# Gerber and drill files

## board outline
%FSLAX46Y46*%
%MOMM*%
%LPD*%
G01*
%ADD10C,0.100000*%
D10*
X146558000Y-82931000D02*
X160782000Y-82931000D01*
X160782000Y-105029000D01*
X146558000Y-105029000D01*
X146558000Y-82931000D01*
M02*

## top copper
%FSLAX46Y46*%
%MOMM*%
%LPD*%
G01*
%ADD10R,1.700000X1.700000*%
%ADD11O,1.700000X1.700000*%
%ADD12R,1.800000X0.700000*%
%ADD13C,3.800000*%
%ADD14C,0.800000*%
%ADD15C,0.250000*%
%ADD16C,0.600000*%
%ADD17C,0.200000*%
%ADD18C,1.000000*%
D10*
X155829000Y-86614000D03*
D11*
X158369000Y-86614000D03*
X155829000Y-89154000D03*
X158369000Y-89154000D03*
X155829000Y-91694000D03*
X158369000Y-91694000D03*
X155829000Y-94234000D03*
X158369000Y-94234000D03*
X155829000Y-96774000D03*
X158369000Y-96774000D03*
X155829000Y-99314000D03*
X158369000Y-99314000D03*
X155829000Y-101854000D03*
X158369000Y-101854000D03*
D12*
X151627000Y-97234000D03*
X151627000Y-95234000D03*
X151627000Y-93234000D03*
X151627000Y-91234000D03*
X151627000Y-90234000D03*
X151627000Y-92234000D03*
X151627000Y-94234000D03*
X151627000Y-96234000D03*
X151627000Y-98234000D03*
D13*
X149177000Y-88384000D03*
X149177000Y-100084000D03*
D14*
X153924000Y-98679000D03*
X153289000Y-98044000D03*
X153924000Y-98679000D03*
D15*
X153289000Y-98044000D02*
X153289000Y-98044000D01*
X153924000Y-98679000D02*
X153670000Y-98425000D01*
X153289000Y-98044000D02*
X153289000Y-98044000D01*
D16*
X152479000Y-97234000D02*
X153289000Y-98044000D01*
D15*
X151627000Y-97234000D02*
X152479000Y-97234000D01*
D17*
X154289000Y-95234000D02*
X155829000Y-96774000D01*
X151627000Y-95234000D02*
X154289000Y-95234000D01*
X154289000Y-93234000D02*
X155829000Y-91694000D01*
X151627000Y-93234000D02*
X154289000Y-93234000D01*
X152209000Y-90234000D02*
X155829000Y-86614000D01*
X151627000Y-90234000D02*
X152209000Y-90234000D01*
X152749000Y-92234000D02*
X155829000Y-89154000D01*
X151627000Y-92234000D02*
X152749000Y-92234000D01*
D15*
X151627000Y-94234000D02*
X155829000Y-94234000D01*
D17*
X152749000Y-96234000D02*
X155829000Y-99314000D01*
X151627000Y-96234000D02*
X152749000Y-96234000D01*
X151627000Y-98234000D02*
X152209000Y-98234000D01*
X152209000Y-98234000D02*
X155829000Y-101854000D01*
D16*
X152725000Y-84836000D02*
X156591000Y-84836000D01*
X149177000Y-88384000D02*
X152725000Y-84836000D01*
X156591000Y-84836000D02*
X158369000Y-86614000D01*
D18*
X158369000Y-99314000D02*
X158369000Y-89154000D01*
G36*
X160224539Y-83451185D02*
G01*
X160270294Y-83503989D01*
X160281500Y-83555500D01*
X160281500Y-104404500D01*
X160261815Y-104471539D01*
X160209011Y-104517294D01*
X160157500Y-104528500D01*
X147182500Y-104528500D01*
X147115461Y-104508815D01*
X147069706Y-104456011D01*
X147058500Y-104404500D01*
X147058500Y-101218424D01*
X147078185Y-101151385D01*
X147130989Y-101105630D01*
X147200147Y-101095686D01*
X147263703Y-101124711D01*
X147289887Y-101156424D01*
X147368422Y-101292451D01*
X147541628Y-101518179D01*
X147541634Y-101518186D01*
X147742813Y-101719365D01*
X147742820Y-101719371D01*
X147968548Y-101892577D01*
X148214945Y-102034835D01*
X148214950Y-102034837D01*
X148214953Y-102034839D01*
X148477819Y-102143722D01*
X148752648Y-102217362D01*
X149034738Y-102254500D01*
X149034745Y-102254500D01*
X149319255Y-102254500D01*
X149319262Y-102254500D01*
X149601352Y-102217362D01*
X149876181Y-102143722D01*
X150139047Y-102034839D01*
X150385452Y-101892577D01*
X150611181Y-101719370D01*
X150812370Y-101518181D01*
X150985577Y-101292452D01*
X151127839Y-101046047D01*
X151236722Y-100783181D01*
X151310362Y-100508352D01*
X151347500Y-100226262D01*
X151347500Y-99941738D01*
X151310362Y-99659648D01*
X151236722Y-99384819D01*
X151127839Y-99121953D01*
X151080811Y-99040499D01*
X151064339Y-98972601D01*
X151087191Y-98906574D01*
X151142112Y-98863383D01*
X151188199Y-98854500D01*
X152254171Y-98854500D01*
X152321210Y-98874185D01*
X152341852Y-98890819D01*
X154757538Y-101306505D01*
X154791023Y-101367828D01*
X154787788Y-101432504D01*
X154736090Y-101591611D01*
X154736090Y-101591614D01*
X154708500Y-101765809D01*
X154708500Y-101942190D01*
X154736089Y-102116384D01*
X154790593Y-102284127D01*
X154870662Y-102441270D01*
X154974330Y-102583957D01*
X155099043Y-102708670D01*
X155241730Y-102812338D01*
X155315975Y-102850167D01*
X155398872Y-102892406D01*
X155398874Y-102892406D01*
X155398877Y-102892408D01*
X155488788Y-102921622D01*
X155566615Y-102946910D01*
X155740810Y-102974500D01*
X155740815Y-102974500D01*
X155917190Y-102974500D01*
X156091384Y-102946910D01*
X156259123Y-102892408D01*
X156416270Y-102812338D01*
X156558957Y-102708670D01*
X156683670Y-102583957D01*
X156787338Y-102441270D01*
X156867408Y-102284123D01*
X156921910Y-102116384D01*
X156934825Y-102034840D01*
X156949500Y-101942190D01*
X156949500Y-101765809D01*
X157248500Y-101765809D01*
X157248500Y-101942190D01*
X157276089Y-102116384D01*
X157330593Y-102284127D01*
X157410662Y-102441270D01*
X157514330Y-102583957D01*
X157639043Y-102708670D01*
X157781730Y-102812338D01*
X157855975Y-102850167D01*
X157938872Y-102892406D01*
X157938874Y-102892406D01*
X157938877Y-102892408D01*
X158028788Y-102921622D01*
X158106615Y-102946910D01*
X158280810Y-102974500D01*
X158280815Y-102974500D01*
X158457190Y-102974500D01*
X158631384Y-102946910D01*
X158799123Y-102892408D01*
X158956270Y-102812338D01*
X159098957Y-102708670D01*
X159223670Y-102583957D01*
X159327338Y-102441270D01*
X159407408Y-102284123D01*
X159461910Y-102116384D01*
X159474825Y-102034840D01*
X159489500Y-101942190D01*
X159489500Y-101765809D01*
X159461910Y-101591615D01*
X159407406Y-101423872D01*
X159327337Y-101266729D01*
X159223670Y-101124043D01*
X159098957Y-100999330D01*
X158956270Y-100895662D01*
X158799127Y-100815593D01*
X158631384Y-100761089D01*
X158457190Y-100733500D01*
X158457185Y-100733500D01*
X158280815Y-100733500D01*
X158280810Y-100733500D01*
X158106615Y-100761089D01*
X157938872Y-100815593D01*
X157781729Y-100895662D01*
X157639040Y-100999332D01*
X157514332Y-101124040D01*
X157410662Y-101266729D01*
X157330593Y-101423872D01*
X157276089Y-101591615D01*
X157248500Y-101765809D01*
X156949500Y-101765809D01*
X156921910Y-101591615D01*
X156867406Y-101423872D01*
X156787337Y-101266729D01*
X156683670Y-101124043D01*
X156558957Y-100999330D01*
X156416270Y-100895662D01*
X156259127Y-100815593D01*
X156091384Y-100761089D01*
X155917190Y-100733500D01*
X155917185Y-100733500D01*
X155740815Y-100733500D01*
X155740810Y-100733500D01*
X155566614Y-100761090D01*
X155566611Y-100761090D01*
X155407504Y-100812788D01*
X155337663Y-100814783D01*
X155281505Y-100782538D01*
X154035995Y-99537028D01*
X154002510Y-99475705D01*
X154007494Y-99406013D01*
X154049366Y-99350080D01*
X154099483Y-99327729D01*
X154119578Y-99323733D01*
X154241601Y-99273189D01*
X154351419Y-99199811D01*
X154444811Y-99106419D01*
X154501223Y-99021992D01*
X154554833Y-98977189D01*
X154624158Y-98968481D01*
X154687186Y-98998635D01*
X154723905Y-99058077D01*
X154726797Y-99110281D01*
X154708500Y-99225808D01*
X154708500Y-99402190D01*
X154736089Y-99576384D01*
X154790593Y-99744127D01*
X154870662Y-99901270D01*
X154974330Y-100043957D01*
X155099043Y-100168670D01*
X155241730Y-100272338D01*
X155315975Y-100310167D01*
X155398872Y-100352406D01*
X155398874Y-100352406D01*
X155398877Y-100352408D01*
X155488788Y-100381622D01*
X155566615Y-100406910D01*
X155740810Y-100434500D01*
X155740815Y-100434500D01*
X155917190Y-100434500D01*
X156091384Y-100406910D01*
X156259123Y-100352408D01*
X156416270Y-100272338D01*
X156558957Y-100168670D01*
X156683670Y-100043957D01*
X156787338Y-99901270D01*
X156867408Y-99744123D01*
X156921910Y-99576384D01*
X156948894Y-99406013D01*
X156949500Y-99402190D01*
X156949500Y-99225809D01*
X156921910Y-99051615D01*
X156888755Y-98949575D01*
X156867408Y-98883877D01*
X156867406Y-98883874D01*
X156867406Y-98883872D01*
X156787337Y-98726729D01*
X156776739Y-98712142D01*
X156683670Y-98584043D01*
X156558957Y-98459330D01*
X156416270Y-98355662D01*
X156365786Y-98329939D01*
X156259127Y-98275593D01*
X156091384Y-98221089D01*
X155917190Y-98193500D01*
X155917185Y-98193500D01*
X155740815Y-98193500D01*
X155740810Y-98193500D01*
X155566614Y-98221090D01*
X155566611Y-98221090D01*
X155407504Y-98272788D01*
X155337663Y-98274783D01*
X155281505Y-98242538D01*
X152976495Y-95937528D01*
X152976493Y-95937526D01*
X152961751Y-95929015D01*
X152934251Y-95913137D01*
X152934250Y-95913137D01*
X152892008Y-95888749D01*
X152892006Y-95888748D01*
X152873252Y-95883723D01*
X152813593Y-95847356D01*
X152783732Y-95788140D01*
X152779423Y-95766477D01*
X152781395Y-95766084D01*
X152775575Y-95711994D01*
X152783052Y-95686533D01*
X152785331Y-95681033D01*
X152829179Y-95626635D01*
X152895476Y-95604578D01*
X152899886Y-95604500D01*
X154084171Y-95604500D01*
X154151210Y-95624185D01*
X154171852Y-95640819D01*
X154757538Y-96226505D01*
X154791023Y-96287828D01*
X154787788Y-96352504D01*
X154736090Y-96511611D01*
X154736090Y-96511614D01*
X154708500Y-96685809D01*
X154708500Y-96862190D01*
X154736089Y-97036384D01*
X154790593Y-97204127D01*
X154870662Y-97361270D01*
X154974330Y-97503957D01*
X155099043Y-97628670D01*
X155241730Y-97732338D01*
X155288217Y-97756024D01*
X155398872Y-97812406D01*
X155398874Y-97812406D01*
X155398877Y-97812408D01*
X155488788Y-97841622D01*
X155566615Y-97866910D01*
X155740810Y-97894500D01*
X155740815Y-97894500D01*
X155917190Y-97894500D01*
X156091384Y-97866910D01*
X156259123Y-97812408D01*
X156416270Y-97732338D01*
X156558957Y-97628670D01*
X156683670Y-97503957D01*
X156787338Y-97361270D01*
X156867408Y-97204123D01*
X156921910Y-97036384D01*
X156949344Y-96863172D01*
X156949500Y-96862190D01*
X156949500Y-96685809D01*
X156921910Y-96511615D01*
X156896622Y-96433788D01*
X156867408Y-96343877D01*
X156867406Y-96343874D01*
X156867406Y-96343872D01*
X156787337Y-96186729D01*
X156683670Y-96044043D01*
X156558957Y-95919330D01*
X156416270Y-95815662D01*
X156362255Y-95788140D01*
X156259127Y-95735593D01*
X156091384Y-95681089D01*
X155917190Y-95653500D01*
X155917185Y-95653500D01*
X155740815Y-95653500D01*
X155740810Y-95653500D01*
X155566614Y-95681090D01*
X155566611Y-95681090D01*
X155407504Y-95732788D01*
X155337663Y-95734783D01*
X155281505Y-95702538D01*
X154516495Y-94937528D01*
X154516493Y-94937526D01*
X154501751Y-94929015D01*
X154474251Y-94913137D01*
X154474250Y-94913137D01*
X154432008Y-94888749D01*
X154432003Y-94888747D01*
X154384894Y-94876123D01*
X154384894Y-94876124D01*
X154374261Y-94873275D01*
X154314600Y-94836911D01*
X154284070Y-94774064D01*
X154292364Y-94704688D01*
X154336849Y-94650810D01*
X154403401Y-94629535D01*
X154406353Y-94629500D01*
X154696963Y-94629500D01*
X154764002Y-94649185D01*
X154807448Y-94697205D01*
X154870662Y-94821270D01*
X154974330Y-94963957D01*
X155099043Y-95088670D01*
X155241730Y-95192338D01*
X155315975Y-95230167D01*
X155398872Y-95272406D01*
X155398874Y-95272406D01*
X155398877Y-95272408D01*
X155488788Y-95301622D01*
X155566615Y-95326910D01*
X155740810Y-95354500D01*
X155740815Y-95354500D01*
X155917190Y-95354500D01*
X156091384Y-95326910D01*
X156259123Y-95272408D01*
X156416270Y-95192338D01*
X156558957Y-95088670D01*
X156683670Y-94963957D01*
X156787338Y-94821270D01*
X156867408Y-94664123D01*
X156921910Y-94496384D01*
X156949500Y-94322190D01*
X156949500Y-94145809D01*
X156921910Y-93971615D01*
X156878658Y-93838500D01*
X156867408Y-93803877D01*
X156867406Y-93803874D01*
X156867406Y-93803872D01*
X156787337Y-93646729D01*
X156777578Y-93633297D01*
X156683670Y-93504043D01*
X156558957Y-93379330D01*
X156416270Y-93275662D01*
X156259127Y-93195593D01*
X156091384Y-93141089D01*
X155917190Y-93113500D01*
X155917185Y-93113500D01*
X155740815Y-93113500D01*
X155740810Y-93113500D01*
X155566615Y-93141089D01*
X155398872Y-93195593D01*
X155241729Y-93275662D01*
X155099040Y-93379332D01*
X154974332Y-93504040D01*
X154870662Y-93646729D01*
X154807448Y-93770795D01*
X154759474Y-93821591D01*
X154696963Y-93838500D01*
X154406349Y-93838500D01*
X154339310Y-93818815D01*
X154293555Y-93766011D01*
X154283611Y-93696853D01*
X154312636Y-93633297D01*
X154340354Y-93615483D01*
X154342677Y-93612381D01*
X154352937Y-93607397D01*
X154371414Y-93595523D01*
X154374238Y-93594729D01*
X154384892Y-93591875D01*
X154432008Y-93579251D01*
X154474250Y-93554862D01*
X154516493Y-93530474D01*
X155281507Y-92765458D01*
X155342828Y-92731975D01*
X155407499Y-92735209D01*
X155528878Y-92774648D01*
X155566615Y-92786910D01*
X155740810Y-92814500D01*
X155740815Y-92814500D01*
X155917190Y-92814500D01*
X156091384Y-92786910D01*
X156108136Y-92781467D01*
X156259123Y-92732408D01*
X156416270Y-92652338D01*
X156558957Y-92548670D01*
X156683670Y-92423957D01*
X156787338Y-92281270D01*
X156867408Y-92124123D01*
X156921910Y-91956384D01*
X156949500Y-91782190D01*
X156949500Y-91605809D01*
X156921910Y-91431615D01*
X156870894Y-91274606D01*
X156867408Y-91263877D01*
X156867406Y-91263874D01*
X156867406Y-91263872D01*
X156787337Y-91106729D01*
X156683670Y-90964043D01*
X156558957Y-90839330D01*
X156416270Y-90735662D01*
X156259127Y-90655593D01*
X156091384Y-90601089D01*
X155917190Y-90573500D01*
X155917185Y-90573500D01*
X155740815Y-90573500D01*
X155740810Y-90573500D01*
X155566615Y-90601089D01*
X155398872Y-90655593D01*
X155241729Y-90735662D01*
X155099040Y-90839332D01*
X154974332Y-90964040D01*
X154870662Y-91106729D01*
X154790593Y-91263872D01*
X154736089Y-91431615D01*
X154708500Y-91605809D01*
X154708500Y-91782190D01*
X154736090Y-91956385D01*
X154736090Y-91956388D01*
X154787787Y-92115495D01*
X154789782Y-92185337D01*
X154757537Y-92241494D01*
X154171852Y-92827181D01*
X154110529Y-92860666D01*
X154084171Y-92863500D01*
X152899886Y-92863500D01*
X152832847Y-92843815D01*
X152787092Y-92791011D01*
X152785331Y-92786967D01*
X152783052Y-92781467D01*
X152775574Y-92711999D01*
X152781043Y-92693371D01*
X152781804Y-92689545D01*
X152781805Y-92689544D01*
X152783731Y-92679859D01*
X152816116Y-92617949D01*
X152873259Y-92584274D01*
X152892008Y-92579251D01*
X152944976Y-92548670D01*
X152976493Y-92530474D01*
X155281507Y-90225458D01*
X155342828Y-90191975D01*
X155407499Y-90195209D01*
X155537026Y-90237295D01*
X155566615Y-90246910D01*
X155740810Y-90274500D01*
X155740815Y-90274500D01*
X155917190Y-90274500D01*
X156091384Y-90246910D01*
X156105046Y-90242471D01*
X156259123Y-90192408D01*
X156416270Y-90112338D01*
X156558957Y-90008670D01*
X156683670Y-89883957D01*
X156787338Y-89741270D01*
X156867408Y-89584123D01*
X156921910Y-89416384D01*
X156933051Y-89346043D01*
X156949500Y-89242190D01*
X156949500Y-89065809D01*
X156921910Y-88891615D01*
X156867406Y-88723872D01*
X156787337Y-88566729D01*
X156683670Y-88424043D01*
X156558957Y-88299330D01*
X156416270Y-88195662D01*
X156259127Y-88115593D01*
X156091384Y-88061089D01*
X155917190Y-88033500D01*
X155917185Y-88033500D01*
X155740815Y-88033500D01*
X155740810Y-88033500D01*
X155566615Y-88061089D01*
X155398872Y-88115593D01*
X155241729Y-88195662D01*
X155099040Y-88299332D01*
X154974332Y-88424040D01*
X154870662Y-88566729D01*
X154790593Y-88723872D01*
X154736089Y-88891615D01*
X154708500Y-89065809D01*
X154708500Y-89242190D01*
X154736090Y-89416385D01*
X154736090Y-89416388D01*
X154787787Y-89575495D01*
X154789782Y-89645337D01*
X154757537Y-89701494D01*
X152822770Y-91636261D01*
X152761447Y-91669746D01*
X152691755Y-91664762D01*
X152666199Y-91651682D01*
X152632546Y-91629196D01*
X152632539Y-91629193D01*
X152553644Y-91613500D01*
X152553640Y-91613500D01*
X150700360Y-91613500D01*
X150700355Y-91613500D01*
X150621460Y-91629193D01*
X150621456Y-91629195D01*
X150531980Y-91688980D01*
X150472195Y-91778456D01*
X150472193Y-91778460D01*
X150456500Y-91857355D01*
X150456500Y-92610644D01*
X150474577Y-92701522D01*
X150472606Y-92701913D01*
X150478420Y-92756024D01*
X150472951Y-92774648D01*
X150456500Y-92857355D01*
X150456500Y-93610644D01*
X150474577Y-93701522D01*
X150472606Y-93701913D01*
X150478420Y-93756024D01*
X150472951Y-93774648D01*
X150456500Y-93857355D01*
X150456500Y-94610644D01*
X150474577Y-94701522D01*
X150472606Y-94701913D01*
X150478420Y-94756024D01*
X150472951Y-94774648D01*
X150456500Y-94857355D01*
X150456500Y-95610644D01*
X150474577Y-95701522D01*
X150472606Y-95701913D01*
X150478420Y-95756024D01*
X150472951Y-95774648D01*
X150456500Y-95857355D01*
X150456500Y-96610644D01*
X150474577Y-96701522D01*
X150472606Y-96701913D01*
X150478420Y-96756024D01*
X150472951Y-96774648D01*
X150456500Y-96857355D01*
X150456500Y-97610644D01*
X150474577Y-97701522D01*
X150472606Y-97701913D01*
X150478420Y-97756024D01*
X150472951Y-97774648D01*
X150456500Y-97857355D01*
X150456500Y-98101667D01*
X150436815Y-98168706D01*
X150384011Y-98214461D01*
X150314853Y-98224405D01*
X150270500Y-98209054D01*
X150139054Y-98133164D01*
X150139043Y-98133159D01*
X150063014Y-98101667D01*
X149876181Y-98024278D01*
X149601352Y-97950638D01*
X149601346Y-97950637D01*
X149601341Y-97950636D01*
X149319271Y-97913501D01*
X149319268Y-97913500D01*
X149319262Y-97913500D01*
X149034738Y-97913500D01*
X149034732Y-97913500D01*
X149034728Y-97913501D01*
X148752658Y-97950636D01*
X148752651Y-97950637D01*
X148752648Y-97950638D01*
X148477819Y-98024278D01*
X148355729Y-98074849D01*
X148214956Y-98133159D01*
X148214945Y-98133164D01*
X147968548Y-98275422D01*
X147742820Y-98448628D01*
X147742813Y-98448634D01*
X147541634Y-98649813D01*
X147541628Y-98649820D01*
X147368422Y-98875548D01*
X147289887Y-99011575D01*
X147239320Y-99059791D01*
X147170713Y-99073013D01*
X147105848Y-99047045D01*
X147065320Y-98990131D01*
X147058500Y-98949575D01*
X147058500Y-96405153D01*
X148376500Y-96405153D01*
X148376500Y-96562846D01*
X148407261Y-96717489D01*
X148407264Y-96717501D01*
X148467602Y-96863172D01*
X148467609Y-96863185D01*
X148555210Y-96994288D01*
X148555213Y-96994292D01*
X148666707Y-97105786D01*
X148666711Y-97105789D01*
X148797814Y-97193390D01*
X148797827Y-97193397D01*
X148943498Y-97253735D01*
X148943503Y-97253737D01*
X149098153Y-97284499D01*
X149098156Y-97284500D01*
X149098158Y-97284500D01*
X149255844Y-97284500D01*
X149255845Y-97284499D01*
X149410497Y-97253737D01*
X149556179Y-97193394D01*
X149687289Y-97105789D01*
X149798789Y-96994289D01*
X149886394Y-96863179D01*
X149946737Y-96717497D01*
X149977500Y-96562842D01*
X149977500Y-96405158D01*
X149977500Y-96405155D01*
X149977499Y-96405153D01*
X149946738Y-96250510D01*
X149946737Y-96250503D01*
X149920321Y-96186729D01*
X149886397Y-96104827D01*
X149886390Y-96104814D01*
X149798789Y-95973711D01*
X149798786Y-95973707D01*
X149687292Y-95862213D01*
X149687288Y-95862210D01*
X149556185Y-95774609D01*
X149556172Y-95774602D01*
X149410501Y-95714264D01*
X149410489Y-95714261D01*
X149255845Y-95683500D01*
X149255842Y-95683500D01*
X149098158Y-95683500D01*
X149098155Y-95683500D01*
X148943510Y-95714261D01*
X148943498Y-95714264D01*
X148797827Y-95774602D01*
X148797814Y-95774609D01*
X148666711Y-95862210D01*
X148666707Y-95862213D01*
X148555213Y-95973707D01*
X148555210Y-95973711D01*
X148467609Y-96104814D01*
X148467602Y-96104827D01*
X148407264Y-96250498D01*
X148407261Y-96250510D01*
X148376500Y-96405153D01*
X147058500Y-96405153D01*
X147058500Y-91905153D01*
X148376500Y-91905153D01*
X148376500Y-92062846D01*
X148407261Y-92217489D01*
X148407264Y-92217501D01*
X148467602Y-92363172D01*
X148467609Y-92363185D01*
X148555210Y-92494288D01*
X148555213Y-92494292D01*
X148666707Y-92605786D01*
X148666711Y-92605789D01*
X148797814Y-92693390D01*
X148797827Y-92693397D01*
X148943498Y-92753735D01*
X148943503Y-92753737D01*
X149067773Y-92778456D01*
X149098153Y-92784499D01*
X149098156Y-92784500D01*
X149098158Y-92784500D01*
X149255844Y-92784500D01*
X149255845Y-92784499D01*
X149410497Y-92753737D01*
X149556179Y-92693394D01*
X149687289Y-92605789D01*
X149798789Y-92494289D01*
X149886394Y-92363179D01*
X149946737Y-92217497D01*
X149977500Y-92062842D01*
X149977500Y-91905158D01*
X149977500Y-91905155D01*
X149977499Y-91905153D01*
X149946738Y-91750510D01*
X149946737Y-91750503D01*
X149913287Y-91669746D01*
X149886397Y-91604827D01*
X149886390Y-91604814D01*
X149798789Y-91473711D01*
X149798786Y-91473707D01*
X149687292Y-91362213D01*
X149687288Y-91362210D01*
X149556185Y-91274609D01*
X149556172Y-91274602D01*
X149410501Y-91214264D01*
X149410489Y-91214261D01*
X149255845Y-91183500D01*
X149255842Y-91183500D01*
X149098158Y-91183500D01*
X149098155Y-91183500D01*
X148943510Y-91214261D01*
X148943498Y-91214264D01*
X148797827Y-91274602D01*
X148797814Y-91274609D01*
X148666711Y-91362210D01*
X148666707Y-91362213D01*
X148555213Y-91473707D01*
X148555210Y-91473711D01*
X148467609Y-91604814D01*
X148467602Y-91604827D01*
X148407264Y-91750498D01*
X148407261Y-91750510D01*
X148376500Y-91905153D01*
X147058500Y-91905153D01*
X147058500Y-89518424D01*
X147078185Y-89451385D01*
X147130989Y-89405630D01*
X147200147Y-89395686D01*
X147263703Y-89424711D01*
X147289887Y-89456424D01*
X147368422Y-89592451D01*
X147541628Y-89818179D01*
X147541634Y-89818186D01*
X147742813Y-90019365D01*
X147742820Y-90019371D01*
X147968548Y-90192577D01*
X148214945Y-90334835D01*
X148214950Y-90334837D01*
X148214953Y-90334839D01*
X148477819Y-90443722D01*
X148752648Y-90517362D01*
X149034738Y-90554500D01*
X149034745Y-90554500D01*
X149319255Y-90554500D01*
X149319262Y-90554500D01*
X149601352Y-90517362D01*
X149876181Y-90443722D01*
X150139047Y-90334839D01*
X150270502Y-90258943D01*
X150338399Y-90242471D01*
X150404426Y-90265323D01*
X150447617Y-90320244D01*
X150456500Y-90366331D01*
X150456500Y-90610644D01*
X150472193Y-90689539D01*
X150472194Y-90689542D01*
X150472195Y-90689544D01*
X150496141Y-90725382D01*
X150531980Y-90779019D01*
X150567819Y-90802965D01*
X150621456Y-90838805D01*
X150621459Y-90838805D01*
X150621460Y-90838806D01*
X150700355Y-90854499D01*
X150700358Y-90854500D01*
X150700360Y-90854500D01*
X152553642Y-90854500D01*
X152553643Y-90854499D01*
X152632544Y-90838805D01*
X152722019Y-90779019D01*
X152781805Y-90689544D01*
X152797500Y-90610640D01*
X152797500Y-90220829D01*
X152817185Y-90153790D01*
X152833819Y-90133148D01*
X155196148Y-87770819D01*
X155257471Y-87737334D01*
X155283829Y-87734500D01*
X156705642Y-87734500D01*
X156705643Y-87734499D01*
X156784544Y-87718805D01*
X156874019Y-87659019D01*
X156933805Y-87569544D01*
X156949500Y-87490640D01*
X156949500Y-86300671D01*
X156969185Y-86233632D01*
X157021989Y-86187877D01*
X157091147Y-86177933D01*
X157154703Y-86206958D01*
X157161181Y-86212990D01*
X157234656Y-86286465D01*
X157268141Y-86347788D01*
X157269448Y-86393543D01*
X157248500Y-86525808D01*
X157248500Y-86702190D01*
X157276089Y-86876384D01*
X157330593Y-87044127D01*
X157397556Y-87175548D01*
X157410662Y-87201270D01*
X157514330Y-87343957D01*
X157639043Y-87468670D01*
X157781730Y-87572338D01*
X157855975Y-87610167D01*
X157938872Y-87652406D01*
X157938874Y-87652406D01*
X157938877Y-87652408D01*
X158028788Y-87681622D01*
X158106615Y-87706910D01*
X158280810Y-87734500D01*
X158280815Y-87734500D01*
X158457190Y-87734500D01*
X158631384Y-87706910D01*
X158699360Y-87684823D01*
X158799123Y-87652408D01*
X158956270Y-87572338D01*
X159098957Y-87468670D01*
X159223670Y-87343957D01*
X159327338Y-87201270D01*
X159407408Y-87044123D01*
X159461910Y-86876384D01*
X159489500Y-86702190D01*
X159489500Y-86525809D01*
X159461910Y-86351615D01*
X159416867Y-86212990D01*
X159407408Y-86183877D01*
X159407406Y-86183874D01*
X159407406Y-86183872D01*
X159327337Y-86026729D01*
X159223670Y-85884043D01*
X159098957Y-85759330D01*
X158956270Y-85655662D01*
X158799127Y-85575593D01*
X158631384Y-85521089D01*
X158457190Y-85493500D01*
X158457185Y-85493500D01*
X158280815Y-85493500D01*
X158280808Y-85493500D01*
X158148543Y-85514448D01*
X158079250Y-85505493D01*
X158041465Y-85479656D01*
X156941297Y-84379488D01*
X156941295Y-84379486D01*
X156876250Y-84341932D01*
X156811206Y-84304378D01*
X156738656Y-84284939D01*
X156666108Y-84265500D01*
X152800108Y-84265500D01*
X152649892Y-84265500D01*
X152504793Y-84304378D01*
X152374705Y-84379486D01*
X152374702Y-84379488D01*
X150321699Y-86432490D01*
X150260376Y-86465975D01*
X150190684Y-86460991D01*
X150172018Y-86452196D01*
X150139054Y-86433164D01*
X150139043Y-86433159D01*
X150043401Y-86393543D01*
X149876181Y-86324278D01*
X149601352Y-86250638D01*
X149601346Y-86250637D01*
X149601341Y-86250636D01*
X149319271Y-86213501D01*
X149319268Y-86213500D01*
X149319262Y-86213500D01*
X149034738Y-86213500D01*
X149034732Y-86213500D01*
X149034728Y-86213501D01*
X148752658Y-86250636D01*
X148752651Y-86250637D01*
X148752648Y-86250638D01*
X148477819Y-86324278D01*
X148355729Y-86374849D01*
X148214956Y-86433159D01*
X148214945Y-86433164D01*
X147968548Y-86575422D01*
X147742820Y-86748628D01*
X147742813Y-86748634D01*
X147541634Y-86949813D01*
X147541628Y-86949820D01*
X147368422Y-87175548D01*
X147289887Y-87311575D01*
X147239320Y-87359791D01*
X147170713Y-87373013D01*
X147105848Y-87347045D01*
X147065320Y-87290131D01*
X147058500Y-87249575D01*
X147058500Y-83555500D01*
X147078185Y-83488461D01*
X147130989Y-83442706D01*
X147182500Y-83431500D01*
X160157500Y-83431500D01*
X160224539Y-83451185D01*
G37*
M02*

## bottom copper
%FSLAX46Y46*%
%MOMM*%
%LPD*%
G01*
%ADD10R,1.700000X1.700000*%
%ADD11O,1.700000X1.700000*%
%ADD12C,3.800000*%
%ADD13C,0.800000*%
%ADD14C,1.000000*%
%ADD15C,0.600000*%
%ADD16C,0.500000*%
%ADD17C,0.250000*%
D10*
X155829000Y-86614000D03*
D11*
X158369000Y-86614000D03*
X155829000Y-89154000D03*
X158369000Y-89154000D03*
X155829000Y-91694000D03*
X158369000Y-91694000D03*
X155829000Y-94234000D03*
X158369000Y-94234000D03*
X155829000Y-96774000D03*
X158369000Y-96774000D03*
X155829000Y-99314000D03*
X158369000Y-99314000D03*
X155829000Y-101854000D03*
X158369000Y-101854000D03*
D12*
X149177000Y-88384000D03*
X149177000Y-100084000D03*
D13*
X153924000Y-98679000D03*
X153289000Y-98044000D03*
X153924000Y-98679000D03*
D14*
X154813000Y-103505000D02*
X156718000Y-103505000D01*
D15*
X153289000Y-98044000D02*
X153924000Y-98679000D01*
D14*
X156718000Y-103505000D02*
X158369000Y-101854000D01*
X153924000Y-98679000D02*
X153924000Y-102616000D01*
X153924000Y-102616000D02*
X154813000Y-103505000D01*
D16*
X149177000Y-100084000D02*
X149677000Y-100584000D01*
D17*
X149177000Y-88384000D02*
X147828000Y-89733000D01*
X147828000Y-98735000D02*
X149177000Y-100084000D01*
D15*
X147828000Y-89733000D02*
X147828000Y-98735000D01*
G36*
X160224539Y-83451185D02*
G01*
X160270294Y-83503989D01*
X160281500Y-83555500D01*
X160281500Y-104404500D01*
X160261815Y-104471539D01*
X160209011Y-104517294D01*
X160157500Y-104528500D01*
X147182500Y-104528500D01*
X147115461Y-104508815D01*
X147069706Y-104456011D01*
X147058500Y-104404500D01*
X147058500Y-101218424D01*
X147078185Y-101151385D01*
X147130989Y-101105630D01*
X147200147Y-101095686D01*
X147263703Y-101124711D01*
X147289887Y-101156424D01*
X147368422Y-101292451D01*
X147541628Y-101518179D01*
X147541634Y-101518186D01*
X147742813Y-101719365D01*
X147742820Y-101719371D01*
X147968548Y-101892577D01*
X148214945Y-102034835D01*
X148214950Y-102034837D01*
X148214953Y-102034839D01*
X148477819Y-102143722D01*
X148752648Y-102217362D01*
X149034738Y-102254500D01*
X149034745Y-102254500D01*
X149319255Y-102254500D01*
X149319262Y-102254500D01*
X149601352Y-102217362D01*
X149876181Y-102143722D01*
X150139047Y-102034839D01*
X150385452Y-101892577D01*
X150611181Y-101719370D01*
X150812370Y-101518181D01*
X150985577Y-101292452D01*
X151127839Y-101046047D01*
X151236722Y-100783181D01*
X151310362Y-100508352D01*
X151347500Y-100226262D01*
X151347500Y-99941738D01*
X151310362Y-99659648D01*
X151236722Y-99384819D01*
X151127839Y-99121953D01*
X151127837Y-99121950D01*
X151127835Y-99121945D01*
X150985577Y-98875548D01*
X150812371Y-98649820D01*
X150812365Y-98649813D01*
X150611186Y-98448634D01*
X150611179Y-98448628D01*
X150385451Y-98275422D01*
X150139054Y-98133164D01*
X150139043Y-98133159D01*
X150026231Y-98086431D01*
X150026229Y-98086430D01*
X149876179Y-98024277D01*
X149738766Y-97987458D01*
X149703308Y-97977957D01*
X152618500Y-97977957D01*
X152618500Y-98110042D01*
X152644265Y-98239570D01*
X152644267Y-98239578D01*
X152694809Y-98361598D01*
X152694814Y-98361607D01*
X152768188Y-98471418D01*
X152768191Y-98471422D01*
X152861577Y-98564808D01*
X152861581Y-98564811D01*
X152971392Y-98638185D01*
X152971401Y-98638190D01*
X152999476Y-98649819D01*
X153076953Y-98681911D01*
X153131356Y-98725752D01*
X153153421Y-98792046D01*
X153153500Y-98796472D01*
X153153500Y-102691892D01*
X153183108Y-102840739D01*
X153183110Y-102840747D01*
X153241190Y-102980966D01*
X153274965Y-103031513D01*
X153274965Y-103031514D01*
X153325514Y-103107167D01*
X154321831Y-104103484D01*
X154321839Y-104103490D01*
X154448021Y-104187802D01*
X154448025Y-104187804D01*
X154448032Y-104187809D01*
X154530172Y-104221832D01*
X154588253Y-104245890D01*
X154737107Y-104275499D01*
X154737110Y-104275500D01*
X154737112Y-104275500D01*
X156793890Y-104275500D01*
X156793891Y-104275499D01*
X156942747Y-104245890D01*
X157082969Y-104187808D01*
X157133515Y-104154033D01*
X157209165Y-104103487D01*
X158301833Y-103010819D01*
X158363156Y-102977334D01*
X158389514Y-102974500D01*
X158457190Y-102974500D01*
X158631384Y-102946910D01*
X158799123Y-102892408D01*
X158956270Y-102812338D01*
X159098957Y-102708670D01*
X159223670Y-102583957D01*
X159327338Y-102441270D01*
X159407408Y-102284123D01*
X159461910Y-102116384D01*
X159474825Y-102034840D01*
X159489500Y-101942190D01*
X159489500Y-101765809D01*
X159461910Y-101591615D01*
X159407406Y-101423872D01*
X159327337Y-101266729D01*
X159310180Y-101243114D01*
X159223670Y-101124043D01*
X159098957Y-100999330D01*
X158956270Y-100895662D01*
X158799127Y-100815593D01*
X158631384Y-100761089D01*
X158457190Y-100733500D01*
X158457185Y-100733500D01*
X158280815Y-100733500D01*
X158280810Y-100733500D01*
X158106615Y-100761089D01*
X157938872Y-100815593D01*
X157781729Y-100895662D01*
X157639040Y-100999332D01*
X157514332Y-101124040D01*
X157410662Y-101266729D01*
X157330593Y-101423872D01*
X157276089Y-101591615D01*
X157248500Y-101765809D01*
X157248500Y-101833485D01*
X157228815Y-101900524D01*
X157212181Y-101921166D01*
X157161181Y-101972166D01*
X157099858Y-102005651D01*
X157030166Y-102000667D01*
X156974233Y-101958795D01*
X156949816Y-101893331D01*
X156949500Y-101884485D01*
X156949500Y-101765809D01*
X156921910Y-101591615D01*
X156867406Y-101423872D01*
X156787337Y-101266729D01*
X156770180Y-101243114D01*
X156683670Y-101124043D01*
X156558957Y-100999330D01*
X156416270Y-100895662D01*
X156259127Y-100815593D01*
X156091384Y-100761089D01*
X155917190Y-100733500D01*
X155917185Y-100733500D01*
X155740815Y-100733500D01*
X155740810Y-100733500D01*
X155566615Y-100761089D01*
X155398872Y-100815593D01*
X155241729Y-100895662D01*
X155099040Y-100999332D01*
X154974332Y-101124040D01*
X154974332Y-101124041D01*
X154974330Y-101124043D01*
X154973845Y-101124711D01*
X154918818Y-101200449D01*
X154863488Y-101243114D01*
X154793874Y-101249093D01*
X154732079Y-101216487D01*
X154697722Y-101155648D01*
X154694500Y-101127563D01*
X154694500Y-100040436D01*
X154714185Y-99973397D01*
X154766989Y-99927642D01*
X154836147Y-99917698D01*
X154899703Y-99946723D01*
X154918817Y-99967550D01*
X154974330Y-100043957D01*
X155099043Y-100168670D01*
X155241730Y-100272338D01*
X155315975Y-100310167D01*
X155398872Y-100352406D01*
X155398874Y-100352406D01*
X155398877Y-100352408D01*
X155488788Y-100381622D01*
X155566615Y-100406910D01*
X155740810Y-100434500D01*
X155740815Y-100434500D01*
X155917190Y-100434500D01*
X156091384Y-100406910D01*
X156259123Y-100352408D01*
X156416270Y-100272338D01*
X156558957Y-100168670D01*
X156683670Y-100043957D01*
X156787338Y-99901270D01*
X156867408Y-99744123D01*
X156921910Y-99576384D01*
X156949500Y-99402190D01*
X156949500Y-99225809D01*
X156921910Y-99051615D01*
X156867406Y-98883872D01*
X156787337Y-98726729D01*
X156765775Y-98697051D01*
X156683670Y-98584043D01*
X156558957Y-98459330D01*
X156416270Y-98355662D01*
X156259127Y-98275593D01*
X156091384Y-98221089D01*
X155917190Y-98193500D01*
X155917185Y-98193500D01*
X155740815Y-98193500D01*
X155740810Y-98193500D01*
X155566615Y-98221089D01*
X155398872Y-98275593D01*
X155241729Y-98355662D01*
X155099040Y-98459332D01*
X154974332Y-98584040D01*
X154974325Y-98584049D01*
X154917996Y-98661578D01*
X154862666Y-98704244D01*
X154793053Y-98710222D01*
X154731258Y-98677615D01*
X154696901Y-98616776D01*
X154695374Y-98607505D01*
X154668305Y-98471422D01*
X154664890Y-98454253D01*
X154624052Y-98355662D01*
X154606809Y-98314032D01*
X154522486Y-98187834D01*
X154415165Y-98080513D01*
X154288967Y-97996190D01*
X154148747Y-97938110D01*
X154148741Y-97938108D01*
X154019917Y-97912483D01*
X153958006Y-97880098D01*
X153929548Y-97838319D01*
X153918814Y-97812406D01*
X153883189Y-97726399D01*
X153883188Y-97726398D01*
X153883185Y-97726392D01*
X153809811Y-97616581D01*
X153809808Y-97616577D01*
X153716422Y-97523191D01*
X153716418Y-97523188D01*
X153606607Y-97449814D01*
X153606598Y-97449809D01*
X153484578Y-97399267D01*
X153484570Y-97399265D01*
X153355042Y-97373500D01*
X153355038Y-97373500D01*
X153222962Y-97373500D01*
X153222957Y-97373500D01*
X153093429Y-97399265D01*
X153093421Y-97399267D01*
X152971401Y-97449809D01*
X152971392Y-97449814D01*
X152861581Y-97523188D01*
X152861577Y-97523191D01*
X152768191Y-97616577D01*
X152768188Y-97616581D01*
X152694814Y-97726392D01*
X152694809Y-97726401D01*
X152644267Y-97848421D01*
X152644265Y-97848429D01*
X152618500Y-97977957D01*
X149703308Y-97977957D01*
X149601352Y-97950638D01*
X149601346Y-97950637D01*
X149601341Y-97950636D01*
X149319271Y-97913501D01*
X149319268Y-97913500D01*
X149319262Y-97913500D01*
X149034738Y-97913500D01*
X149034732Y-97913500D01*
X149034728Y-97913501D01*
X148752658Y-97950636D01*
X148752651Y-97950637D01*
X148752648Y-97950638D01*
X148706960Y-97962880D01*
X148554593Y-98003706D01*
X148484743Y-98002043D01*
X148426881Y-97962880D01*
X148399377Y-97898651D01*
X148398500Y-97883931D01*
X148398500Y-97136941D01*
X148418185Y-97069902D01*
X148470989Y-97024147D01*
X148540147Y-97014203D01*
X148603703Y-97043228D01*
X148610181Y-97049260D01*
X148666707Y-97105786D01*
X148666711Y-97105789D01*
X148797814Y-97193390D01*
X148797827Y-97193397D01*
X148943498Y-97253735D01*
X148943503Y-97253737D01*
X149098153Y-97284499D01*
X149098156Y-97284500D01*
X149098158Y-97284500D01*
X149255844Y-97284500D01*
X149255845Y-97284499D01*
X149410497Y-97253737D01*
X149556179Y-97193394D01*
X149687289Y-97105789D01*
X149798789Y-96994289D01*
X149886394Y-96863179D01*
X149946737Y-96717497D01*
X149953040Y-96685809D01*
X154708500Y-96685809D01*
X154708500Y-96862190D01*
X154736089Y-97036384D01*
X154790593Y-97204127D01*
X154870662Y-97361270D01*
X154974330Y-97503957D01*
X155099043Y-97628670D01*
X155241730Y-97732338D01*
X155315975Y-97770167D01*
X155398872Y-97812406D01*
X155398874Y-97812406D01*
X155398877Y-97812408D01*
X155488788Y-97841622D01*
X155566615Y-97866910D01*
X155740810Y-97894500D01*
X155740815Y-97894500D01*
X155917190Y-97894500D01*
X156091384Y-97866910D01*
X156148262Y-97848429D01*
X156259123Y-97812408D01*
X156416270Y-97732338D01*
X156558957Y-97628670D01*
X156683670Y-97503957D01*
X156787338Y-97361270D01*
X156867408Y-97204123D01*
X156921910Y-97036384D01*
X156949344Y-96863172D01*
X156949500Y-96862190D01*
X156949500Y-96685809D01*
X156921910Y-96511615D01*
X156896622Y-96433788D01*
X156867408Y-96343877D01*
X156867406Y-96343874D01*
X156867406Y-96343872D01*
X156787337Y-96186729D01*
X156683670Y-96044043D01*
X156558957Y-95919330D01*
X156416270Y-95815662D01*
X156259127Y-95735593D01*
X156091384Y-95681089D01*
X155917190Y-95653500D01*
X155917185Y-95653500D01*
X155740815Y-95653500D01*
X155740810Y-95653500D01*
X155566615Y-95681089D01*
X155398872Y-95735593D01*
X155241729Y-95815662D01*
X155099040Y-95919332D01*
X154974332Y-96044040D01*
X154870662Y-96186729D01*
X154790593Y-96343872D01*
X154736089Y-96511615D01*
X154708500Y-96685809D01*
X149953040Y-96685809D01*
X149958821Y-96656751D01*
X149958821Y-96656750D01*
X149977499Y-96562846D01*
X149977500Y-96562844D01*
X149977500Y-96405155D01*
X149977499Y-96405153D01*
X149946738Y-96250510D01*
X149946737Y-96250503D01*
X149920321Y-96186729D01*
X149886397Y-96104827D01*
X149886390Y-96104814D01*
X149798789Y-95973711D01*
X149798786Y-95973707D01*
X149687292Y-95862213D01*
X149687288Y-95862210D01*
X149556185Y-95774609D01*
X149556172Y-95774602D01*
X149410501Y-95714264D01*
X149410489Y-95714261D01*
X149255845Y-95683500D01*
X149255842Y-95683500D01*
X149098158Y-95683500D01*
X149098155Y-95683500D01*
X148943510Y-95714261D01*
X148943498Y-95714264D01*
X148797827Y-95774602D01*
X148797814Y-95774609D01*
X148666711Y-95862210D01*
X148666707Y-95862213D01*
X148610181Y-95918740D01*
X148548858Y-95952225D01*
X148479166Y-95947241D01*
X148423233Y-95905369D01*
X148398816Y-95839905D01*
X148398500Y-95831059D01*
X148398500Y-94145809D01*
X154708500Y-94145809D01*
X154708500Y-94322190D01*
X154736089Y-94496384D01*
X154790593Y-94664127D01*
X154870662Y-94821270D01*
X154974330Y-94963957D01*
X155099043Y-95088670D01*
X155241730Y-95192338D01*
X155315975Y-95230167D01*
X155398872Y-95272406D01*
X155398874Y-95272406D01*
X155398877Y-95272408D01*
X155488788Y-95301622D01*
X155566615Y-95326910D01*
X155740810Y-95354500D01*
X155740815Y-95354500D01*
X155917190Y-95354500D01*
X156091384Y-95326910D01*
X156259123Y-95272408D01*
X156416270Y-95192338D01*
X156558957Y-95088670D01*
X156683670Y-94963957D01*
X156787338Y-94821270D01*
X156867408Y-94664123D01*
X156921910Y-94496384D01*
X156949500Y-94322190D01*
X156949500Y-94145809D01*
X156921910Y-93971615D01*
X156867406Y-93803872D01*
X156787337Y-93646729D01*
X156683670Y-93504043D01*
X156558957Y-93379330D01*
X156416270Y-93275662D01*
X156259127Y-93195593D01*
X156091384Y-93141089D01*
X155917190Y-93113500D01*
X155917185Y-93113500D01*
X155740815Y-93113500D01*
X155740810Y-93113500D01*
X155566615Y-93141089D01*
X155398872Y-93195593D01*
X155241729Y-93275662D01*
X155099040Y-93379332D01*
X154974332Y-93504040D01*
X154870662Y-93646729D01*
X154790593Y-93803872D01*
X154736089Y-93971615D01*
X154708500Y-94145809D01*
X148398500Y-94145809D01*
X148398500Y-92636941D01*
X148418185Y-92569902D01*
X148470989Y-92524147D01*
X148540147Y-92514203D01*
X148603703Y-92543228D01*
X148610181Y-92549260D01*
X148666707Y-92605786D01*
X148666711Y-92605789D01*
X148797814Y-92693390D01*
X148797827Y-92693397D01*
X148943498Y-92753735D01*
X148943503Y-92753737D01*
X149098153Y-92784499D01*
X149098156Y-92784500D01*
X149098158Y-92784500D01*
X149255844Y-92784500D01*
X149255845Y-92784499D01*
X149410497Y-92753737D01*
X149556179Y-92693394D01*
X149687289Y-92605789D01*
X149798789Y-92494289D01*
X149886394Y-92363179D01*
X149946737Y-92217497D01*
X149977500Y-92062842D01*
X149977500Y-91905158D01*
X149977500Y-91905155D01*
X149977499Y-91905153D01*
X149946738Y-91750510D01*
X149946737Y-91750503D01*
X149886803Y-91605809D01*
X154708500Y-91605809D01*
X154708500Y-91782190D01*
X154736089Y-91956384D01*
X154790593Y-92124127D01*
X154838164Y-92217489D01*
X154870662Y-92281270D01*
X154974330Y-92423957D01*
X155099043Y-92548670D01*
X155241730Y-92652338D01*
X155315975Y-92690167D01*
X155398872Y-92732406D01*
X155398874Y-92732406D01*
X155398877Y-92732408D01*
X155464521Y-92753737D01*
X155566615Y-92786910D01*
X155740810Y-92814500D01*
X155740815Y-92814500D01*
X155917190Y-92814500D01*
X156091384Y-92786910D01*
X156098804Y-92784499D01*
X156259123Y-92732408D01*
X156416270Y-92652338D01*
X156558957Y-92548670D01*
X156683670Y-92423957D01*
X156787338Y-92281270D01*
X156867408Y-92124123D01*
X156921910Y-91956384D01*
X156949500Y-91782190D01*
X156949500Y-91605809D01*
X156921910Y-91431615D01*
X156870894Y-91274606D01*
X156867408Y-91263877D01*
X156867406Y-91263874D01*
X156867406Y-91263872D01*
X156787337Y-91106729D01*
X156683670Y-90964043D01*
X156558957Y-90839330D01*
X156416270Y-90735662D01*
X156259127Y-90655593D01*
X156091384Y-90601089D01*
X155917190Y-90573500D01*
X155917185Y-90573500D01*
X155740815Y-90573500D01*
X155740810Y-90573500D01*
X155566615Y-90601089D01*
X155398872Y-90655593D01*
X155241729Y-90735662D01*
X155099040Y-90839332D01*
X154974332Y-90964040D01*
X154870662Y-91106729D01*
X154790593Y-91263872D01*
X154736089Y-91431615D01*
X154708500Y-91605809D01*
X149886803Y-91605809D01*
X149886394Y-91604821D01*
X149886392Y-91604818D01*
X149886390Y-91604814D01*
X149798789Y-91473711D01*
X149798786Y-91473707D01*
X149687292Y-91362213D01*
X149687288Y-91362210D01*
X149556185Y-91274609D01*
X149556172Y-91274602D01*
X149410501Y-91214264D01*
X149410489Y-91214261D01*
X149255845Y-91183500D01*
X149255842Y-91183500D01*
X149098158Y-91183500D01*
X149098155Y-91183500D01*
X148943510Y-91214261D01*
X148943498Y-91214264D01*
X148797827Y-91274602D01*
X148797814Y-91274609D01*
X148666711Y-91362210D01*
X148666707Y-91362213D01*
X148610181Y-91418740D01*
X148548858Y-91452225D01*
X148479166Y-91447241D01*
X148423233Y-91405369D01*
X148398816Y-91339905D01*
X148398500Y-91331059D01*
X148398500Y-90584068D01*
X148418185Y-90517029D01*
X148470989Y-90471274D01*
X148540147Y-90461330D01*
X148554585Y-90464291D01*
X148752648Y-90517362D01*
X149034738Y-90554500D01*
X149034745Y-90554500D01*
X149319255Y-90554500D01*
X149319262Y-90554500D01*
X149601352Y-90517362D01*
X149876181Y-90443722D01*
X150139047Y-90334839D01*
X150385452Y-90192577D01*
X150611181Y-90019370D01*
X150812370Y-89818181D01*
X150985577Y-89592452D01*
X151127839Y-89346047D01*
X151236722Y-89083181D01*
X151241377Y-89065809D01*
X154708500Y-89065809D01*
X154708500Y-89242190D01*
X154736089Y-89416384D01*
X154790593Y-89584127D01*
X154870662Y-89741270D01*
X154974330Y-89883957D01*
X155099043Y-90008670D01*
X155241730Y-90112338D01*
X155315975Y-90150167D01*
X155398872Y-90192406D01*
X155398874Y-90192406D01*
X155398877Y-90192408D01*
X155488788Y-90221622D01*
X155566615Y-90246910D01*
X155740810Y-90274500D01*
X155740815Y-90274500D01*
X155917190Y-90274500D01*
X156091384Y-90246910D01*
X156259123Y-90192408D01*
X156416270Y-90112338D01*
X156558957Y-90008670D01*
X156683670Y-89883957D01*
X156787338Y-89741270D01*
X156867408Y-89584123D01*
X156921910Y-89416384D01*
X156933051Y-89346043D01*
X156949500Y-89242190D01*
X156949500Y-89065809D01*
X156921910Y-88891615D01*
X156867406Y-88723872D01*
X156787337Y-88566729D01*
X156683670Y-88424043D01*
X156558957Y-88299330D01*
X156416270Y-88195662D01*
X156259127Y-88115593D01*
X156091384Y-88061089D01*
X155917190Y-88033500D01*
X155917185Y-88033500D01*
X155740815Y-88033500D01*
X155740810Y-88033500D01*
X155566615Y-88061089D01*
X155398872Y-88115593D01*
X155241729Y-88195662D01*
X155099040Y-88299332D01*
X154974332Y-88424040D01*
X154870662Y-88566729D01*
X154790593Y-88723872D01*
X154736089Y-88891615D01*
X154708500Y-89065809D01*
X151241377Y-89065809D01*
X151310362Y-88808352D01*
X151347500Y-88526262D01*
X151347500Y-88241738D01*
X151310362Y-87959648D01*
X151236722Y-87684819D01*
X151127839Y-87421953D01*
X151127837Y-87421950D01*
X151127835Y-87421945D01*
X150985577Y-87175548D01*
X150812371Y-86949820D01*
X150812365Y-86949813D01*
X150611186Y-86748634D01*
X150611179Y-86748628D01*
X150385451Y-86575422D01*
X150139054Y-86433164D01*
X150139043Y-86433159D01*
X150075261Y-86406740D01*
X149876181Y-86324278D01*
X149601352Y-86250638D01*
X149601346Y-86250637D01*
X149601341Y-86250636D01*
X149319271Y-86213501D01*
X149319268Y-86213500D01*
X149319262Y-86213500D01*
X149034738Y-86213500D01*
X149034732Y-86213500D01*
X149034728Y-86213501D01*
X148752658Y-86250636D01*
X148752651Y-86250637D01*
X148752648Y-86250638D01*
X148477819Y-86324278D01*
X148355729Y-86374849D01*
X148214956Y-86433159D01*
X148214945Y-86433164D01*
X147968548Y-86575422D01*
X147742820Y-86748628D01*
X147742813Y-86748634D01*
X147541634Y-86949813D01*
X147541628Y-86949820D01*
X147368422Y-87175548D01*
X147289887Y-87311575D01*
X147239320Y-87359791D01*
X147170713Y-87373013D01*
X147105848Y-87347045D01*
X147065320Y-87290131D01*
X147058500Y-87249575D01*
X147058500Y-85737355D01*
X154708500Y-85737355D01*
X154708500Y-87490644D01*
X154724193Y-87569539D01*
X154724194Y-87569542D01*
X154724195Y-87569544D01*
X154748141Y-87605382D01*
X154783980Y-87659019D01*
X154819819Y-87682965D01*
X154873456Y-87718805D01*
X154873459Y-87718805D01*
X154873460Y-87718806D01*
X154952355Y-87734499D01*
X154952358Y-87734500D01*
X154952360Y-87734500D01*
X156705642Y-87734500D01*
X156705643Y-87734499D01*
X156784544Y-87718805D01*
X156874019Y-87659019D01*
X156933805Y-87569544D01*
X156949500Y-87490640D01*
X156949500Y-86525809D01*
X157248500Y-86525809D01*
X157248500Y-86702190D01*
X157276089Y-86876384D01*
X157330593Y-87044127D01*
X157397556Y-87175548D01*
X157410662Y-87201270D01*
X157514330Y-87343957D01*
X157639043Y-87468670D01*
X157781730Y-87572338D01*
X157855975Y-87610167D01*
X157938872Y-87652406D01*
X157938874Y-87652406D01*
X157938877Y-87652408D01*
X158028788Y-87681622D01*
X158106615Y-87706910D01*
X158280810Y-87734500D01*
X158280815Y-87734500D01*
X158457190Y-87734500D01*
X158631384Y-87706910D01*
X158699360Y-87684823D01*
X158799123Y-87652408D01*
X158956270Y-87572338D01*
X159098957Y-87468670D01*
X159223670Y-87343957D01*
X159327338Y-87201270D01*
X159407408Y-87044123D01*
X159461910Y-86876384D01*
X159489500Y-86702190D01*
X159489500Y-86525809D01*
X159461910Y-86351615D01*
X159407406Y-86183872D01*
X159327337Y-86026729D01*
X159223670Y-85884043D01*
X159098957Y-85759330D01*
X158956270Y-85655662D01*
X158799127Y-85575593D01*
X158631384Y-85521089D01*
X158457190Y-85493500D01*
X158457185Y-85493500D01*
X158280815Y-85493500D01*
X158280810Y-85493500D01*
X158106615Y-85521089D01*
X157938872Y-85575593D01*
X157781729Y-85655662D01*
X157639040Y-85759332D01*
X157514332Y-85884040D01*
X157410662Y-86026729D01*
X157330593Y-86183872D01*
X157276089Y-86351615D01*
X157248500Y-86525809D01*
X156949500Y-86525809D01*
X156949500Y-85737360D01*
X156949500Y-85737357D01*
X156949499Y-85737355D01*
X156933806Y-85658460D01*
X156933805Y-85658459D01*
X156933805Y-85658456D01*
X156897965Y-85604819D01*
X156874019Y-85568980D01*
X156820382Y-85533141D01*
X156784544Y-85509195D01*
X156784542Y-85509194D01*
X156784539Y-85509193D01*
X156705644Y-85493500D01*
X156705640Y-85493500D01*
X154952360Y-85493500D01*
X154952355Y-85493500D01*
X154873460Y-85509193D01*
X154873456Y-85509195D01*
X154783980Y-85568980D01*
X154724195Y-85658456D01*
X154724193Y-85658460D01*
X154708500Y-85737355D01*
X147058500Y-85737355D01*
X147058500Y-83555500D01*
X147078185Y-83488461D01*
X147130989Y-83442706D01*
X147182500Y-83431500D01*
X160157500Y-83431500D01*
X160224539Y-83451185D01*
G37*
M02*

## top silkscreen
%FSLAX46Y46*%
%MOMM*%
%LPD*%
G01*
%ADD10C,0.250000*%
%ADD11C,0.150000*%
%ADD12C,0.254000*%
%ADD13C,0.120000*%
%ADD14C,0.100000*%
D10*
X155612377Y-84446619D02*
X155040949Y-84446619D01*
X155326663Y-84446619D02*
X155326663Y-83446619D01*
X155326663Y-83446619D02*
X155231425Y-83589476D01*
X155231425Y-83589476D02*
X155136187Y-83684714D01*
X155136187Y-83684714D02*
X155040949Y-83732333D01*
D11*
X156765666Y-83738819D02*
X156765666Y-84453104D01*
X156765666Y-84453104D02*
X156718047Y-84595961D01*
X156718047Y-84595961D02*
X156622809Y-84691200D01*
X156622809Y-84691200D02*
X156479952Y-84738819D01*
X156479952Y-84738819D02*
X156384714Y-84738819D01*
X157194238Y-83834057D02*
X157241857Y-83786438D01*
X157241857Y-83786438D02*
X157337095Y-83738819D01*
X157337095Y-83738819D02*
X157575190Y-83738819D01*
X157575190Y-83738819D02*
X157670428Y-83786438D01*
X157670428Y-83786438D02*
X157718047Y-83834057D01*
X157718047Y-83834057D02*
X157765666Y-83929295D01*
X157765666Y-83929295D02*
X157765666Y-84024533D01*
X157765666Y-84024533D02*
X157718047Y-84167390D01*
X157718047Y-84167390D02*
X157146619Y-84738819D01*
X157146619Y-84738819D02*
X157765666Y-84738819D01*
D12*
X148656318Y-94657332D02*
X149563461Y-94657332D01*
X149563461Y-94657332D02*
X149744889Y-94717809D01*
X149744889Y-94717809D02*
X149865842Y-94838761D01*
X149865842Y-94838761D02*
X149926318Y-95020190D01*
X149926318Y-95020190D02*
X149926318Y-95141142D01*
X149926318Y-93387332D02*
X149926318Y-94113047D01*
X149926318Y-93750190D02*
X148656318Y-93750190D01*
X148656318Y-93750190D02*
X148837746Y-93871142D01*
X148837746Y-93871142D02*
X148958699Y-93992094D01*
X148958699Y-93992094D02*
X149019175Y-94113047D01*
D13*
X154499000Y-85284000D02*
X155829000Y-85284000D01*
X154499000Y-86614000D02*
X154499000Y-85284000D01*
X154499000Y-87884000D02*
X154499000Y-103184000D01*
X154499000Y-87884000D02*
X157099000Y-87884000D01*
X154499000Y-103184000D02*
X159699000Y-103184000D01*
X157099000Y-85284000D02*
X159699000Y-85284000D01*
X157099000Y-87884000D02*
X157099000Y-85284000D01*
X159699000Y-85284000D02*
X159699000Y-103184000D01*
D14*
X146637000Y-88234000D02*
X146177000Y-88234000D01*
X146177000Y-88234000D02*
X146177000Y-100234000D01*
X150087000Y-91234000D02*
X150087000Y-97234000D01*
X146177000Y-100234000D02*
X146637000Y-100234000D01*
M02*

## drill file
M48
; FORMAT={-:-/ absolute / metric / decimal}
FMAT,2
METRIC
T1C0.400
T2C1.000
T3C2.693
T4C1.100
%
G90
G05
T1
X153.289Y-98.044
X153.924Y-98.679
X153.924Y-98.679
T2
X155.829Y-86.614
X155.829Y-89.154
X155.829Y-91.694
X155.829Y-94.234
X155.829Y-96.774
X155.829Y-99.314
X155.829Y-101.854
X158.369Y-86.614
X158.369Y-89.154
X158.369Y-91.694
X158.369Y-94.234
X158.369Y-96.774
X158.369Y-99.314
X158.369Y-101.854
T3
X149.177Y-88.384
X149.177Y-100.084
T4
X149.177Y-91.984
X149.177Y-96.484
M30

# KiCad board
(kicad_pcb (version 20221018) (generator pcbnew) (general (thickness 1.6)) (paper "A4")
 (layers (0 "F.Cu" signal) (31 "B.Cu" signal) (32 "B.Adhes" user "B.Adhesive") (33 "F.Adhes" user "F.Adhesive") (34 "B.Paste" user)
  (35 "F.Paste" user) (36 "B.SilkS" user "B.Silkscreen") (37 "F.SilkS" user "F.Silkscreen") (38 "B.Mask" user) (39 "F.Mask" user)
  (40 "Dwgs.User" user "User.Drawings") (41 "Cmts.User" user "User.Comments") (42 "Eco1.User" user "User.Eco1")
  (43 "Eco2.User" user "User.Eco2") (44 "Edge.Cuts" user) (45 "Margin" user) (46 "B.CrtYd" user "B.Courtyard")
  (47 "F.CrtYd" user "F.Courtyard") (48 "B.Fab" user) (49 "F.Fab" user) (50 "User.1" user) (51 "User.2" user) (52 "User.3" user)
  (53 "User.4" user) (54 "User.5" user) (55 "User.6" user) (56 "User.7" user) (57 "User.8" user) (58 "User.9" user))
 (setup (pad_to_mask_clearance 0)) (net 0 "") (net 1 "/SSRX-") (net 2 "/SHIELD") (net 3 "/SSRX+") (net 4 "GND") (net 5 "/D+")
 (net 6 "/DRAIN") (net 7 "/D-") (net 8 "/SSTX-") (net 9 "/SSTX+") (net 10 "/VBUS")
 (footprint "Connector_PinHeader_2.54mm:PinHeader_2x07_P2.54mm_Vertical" (layer "F.Cu") (at 155.829 86.614)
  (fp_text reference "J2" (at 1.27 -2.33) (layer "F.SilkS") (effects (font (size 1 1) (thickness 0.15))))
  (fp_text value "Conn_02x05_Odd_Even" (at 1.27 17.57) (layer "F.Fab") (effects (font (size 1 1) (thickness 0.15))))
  (fp_line (start -1.33 -1.33) (end 0 -1.33) (stroke (width 0.12) (type solid)) (layer "F.SilkS"))
  (fp_line (start -1.33 0) (end -1.33 -1.33) (stroke (width 0.12) (type solid)) (layer "F.SilkS"))
  (fp_line (start -1.33 1.27) (end -1.33 16.57) (stroke (width 0.12) (type solid)) (layer "F.SilkS"))
  (fp_line (start -1.33 1.27) (end 1.27 1.27) (stroke (width 0.12) (type solid)) (layer "F.SilkS"))
  (fp_line (start -1.33 16.57) (end 3.87 16.57) (stroke (width 0.12) (type solid)) (layer "F.SilkS"))
  (fp_line (start 1.27 -1.33) (end 3.87 -1.33) (stroke (width 0.12) (type solid)) (layer "F.SilkS"))
  (fp_line (start 1.27 1.27) (end 1.27 -1.33) (stroke (width 0.12) (type solid)) (layer "F.SilkS"))
  (fp_line (start 3.87 -1.33) (end 3.87 16.57) (stroke (width 0.12) (type solid)) (layer "F.SilkS"))
  (pad "1" thru_hole rect (at 0 0) (size 1.7 1.7) (drill 1) (layers "*.Cu" "*.Mask") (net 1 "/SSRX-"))
  (pad "2" thru_hole oval (at 2.54 0) (size 1.7 1.7) (drill 1) (layers "*.Cu" "*.Mask") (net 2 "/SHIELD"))
  (pad "3" thru_hole oval (at 0 2.54) (size 1.7 1.7) (drill 1) (layers "*.Cu" "*.Mask") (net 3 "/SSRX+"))
  (pad "4" thru_hole oval (at 2.54 2.54) (size 1.7 1.7) (drill 1) (layers "*.Cu" "*.Mask") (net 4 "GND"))
  (pad "5" thru_hole oval (at 0 5.08) (size 1.7 1.7) (drill 1) (layers "*.Cu" "*.Mask") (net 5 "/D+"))
  (pad "6" thru_hole oval (at 2.54 5.08) (size 1.7 1.7) (drill 1) (layers "*.Cu" "*.Mask") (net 4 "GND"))
  (pad "7" thru_hole oval (at 0 7.62) (size 1.7 1.7) (drill 1) (layers "*.Cu" "*.Mask") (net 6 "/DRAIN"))
  (pad "8" thru_hole oval (at 2.54 7.62) (size 1.7 1.7) (drill 1) (layers "*.Cu" "*.Mask") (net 4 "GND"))
  (pad "9" thru_hole oval (at 0 10.16) (size 1.7 1.7) (drill 1) (layers "*.Cu" "*.Mask") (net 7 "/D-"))
  (pad "10" thru_hole oval (at 2.54 10.16) (size 1.7 1.7) (drill 1) (layers "*.Cu" "*.Mask") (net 4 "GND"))
  (pad "11" thru_hole oval (at 0 12.7) (size 1.7 1.7) (drill 1) (layers "*.Cu" "*.Mask") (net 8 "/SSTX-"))
  (pad "12" thru_hole oval (at 2.54 12.7) (size 1.7 1.7) (drill 1) (layers "*.Cu" "*.Mask") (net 4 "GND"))
  (pad "13" thru_hole oval (at 0 15.24) (size 1.7 1.7) (drill 1) (layers "*.Cu" "*.Mask") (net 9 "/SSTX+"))
  (pad "14" thru_hole oval (at 2.54 15.24) (size 1.7 1.7) (drill 1) (layers "*.Cu" "*.Mask") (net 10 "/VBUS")))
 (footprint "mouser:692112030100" (layer "F.Cu") (at 149.352 94.234 -90)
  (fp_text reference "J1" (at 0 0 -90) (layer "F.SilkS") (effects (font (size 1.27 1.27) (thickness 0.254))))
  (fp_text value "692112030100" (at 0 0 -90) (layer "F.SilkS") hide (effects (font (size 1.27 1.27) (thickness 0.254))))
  (fp_line (start -6 2.715) (end -6 3.175) (stroke (width 0.1) (type solid)) (layer "F.SilkS"))
  (fp_line (start -6 3.175) (end 6 3.175) (stroke (width 0.1) (type solid)) (layer "F.SilkS"))
  (fp_line (start -3 -0.735) (end 3 -0.735) (stroke (width 0.1) (type solid)) (layer "F.SilkS"))
  (fp_line (start 6 3.175) (end 6 2.715) (stroke (width 0.1) (type solid)) (layer "F.SilkS"))
  (pad "" np_thru_hole circle (at -2.25 0.175 270) (size 0.001 0.001) (drill 1.1) (layers "*.Cu" "*.Mask"))
  (pad "" np_thru_hole circle (at 2.25 0.175 270) (size 0.001 0.001) (drill 1.1) (layers "*.Cu" "*.Mask"))
  (pad "1" smd rect (at 3 -2.275 270) (size 0.7 1.8) (layers "F.Cu" "F.Paste" "F.Mask") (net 10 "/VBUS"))
  (pad "2" smd rect (at 1 -2.275 270) (size 0.7 1.8) (layers "F.Cu" "F.Paste" "F.Mask") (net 7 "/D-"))
  (pad "3" smd rect (at -1 -2.275 270) (size 0.7 1.8) (layers "F.Cu" "F.Paste" "F.Mask") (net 5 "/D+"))
  (pad "4" smd rect (at -3 -2.275 270) (size 0.7 1.8) (layers "F.Cu" "F.Paste" "F.Mask") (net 4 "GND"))
  (pad "5" smd rect (at -4 -2.275 270) (size 0.7 1.8) (layers "F.Cu" "F.Paste" "F.Mask") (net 1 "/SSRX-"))
  (pad "6" smd rect (at -2 -2.275 270) (size 0.7 1.8) (layers "F.Cu" "F.Paste" "F.Mask") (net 3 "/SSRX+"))
  (pad "7" smd rect (at 0 -2.275 270) (size 0.7 1.8) (layers "F.Cu" "F.Paste" "F.Mask") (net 6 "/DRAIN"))
  (pad "8" smd rect (at 2 -2.275 270) (size 0.7 1.8) (layers "F.Cu" "F.Paste" "F.Mask") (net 8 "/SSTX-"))
  (pad "9" smd rect (at 4 -2.275 270) (size 0.7 1.8) (layers "F.Cu" "F.Paste" "F.Mask") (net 9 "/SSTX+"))
  (pad "10" thru_hole circle (at -5.85 0.175 270) (size 3.8 3.8) (drill 2.6926) (layers "*.Cu" "*.Mask") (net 2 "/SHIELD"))
  (pad "11" thru_hole circle (at 5.85 0.175 270) (size 3.8 3.8) (drill 2.6926) (layers "*.Cu" "*.Mask") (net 2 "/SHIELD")))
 (gr_rect (start 146.558 82.931) (end 160.782 105.029) (stroke (width 0.1) (type solid)) (fill none) (layer "Edge.Cuts"))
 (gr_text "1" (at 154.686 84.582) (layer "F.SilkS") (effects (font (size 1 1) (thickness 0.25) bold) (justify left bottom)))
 (segment (start 153.289 98.044) (end 153.289 98.044) (width 0.25) (layer "F.Cu") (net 10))
 (segment (start 153.924 98.679) (end 153.67 98.425) (width 0.25) (layer "F.Cu") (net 10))
 (segment (start 153.289 98.044) (end 153.289 98.044) (width 0.25) (layer "F.Cu") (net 10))
 (segment (start 152.479 97.234) (end 153.289 98.044) (width 0.6) (layer "F.Cu") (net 10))
 (segment (start 151.627 97.234) (end 152.479 97.234) (width 0.25) (layer "F.Cu") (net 10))
 (via (at 153.924 98.679) (size 0.8) (drill 0.4) (layers "F.Cu" "B.Cu") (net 10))
 (via (at 153.289 98.044) (size 0.8) (drill 0.4) (layers "F.Cu" "B.Cu") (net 10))
 (via (at 153.924 98.679) (size 0.8) (drill 0.4) (layers "F.Cu" "B.Cu") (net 10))
 (segment (start 154.813 103.505) (end 156.718 103.505) (width 1) (layer "B.Cu") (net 10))
 (segment (start 153.289 98.044) (end 153.924 98.679) (width 0.6) (layer "B.Cu") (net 10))
 (segment (start 156.718 103.505) (end 158.369 101.854) (width 1) (layer "B.Cu") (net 10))
 (segment (start 153.924 98.679) (end 153.924 102.616) (width 1) (layer "B.Cu") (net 10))
 (segment (start 153.924 102.616) (end 154.813 103.505) (width 1) (layer "B.Cu") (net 10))
 (segment (start 154.289 95.234) (end 155.829 96.774) (width 0.2) (layer "F.Cu") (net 7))
 (segment (start 151.627 95.234) (end 154.289 95.234) (width 0.2) (layer "F.Cu") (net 7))
 (segment (start 154.289 93.234) (end 155.829 91.694) (width 0.2) (layer "F.Cu") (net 5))
 (segment (start 151.627 93.234) (end 154.289 93.234) (width 0.2) (layer "F.Cu") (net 5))
 (segment (start 152.209 90.234) (end 155.829 86.614) (width 0.2) (layer "F.Cu") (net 1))
 (segment (start 151.627 90.234) (end 152.209 90.234) (width 0.2) (layer "F.Cu") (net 1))
 (segment (start 152.749 92.234) (end 155.829 89.154) (width 0.2) (layer "F.Cu") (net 3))
 (segment (start 151.627 92.234) (end 152.749 92.234) (width 0.2) (layer "F.Cu") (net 3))
 (segment (start 151.627 94.234) (end 155.829 94.234) (width 0.25) (layer "F.Cu") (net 6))
 (segment (start 152.749 96.234) (end 155.829 99.314) (width 0.2) (layer "F.Cu") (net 8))
 (segment (start 151.627 96.234) (end 152.749 96.234) (width 0.2) (layer "F.Cu") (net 8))
 (segment (start 151.627 98.234) (end 152.209 98.234) (width 0.2) (layer "F.Cu") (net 9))
 (segment (start 152.209 98.234) (end 155.829 101.854) (width 0.2) (layer "F.Cu") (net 9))
 (segment (start 152.725 84.836) (end 156.591 84.836) (width 0.6) (layer "F.Cu") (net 2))
 (segment (start 149.177 88.384) (end 152.725 84.836) (width 0.6) (layer "F.Cu") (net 2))
 (segment (start 156.591 84.836) (end 158.369 86.614) (width 0.6) (layer "F.Cu") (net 2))
 (segment (start 149.177 100.084) (end 149.677 100.584) (width 0.5) (layer "B.Cu") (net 2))
 (segment (start 149.177 88.384) (end 147.828 89.733) (width 0.25) (layer "B.Cu") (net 2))
 (segment (start 147.828 98.735) (end 149.177 100.084) (width 0.25) (layer "B.Cu") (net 2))
 (segment (start 147.828 89.733) (end 147.828 98.735) (width 0.6) (layer "B.Cu") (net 2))
 (segment (start 158.369 99.314) (end 158.369 89.154) (width 1) (layer "F.Cu") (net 4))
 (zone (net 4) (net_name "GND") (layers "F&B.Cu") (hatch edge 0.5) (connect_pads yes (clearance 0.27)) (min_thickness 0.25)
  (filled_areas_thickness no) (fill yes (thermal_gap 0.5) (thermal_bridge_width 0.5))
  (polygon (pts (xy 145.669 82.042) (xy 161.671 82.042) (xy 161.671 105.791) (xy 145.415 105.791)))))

